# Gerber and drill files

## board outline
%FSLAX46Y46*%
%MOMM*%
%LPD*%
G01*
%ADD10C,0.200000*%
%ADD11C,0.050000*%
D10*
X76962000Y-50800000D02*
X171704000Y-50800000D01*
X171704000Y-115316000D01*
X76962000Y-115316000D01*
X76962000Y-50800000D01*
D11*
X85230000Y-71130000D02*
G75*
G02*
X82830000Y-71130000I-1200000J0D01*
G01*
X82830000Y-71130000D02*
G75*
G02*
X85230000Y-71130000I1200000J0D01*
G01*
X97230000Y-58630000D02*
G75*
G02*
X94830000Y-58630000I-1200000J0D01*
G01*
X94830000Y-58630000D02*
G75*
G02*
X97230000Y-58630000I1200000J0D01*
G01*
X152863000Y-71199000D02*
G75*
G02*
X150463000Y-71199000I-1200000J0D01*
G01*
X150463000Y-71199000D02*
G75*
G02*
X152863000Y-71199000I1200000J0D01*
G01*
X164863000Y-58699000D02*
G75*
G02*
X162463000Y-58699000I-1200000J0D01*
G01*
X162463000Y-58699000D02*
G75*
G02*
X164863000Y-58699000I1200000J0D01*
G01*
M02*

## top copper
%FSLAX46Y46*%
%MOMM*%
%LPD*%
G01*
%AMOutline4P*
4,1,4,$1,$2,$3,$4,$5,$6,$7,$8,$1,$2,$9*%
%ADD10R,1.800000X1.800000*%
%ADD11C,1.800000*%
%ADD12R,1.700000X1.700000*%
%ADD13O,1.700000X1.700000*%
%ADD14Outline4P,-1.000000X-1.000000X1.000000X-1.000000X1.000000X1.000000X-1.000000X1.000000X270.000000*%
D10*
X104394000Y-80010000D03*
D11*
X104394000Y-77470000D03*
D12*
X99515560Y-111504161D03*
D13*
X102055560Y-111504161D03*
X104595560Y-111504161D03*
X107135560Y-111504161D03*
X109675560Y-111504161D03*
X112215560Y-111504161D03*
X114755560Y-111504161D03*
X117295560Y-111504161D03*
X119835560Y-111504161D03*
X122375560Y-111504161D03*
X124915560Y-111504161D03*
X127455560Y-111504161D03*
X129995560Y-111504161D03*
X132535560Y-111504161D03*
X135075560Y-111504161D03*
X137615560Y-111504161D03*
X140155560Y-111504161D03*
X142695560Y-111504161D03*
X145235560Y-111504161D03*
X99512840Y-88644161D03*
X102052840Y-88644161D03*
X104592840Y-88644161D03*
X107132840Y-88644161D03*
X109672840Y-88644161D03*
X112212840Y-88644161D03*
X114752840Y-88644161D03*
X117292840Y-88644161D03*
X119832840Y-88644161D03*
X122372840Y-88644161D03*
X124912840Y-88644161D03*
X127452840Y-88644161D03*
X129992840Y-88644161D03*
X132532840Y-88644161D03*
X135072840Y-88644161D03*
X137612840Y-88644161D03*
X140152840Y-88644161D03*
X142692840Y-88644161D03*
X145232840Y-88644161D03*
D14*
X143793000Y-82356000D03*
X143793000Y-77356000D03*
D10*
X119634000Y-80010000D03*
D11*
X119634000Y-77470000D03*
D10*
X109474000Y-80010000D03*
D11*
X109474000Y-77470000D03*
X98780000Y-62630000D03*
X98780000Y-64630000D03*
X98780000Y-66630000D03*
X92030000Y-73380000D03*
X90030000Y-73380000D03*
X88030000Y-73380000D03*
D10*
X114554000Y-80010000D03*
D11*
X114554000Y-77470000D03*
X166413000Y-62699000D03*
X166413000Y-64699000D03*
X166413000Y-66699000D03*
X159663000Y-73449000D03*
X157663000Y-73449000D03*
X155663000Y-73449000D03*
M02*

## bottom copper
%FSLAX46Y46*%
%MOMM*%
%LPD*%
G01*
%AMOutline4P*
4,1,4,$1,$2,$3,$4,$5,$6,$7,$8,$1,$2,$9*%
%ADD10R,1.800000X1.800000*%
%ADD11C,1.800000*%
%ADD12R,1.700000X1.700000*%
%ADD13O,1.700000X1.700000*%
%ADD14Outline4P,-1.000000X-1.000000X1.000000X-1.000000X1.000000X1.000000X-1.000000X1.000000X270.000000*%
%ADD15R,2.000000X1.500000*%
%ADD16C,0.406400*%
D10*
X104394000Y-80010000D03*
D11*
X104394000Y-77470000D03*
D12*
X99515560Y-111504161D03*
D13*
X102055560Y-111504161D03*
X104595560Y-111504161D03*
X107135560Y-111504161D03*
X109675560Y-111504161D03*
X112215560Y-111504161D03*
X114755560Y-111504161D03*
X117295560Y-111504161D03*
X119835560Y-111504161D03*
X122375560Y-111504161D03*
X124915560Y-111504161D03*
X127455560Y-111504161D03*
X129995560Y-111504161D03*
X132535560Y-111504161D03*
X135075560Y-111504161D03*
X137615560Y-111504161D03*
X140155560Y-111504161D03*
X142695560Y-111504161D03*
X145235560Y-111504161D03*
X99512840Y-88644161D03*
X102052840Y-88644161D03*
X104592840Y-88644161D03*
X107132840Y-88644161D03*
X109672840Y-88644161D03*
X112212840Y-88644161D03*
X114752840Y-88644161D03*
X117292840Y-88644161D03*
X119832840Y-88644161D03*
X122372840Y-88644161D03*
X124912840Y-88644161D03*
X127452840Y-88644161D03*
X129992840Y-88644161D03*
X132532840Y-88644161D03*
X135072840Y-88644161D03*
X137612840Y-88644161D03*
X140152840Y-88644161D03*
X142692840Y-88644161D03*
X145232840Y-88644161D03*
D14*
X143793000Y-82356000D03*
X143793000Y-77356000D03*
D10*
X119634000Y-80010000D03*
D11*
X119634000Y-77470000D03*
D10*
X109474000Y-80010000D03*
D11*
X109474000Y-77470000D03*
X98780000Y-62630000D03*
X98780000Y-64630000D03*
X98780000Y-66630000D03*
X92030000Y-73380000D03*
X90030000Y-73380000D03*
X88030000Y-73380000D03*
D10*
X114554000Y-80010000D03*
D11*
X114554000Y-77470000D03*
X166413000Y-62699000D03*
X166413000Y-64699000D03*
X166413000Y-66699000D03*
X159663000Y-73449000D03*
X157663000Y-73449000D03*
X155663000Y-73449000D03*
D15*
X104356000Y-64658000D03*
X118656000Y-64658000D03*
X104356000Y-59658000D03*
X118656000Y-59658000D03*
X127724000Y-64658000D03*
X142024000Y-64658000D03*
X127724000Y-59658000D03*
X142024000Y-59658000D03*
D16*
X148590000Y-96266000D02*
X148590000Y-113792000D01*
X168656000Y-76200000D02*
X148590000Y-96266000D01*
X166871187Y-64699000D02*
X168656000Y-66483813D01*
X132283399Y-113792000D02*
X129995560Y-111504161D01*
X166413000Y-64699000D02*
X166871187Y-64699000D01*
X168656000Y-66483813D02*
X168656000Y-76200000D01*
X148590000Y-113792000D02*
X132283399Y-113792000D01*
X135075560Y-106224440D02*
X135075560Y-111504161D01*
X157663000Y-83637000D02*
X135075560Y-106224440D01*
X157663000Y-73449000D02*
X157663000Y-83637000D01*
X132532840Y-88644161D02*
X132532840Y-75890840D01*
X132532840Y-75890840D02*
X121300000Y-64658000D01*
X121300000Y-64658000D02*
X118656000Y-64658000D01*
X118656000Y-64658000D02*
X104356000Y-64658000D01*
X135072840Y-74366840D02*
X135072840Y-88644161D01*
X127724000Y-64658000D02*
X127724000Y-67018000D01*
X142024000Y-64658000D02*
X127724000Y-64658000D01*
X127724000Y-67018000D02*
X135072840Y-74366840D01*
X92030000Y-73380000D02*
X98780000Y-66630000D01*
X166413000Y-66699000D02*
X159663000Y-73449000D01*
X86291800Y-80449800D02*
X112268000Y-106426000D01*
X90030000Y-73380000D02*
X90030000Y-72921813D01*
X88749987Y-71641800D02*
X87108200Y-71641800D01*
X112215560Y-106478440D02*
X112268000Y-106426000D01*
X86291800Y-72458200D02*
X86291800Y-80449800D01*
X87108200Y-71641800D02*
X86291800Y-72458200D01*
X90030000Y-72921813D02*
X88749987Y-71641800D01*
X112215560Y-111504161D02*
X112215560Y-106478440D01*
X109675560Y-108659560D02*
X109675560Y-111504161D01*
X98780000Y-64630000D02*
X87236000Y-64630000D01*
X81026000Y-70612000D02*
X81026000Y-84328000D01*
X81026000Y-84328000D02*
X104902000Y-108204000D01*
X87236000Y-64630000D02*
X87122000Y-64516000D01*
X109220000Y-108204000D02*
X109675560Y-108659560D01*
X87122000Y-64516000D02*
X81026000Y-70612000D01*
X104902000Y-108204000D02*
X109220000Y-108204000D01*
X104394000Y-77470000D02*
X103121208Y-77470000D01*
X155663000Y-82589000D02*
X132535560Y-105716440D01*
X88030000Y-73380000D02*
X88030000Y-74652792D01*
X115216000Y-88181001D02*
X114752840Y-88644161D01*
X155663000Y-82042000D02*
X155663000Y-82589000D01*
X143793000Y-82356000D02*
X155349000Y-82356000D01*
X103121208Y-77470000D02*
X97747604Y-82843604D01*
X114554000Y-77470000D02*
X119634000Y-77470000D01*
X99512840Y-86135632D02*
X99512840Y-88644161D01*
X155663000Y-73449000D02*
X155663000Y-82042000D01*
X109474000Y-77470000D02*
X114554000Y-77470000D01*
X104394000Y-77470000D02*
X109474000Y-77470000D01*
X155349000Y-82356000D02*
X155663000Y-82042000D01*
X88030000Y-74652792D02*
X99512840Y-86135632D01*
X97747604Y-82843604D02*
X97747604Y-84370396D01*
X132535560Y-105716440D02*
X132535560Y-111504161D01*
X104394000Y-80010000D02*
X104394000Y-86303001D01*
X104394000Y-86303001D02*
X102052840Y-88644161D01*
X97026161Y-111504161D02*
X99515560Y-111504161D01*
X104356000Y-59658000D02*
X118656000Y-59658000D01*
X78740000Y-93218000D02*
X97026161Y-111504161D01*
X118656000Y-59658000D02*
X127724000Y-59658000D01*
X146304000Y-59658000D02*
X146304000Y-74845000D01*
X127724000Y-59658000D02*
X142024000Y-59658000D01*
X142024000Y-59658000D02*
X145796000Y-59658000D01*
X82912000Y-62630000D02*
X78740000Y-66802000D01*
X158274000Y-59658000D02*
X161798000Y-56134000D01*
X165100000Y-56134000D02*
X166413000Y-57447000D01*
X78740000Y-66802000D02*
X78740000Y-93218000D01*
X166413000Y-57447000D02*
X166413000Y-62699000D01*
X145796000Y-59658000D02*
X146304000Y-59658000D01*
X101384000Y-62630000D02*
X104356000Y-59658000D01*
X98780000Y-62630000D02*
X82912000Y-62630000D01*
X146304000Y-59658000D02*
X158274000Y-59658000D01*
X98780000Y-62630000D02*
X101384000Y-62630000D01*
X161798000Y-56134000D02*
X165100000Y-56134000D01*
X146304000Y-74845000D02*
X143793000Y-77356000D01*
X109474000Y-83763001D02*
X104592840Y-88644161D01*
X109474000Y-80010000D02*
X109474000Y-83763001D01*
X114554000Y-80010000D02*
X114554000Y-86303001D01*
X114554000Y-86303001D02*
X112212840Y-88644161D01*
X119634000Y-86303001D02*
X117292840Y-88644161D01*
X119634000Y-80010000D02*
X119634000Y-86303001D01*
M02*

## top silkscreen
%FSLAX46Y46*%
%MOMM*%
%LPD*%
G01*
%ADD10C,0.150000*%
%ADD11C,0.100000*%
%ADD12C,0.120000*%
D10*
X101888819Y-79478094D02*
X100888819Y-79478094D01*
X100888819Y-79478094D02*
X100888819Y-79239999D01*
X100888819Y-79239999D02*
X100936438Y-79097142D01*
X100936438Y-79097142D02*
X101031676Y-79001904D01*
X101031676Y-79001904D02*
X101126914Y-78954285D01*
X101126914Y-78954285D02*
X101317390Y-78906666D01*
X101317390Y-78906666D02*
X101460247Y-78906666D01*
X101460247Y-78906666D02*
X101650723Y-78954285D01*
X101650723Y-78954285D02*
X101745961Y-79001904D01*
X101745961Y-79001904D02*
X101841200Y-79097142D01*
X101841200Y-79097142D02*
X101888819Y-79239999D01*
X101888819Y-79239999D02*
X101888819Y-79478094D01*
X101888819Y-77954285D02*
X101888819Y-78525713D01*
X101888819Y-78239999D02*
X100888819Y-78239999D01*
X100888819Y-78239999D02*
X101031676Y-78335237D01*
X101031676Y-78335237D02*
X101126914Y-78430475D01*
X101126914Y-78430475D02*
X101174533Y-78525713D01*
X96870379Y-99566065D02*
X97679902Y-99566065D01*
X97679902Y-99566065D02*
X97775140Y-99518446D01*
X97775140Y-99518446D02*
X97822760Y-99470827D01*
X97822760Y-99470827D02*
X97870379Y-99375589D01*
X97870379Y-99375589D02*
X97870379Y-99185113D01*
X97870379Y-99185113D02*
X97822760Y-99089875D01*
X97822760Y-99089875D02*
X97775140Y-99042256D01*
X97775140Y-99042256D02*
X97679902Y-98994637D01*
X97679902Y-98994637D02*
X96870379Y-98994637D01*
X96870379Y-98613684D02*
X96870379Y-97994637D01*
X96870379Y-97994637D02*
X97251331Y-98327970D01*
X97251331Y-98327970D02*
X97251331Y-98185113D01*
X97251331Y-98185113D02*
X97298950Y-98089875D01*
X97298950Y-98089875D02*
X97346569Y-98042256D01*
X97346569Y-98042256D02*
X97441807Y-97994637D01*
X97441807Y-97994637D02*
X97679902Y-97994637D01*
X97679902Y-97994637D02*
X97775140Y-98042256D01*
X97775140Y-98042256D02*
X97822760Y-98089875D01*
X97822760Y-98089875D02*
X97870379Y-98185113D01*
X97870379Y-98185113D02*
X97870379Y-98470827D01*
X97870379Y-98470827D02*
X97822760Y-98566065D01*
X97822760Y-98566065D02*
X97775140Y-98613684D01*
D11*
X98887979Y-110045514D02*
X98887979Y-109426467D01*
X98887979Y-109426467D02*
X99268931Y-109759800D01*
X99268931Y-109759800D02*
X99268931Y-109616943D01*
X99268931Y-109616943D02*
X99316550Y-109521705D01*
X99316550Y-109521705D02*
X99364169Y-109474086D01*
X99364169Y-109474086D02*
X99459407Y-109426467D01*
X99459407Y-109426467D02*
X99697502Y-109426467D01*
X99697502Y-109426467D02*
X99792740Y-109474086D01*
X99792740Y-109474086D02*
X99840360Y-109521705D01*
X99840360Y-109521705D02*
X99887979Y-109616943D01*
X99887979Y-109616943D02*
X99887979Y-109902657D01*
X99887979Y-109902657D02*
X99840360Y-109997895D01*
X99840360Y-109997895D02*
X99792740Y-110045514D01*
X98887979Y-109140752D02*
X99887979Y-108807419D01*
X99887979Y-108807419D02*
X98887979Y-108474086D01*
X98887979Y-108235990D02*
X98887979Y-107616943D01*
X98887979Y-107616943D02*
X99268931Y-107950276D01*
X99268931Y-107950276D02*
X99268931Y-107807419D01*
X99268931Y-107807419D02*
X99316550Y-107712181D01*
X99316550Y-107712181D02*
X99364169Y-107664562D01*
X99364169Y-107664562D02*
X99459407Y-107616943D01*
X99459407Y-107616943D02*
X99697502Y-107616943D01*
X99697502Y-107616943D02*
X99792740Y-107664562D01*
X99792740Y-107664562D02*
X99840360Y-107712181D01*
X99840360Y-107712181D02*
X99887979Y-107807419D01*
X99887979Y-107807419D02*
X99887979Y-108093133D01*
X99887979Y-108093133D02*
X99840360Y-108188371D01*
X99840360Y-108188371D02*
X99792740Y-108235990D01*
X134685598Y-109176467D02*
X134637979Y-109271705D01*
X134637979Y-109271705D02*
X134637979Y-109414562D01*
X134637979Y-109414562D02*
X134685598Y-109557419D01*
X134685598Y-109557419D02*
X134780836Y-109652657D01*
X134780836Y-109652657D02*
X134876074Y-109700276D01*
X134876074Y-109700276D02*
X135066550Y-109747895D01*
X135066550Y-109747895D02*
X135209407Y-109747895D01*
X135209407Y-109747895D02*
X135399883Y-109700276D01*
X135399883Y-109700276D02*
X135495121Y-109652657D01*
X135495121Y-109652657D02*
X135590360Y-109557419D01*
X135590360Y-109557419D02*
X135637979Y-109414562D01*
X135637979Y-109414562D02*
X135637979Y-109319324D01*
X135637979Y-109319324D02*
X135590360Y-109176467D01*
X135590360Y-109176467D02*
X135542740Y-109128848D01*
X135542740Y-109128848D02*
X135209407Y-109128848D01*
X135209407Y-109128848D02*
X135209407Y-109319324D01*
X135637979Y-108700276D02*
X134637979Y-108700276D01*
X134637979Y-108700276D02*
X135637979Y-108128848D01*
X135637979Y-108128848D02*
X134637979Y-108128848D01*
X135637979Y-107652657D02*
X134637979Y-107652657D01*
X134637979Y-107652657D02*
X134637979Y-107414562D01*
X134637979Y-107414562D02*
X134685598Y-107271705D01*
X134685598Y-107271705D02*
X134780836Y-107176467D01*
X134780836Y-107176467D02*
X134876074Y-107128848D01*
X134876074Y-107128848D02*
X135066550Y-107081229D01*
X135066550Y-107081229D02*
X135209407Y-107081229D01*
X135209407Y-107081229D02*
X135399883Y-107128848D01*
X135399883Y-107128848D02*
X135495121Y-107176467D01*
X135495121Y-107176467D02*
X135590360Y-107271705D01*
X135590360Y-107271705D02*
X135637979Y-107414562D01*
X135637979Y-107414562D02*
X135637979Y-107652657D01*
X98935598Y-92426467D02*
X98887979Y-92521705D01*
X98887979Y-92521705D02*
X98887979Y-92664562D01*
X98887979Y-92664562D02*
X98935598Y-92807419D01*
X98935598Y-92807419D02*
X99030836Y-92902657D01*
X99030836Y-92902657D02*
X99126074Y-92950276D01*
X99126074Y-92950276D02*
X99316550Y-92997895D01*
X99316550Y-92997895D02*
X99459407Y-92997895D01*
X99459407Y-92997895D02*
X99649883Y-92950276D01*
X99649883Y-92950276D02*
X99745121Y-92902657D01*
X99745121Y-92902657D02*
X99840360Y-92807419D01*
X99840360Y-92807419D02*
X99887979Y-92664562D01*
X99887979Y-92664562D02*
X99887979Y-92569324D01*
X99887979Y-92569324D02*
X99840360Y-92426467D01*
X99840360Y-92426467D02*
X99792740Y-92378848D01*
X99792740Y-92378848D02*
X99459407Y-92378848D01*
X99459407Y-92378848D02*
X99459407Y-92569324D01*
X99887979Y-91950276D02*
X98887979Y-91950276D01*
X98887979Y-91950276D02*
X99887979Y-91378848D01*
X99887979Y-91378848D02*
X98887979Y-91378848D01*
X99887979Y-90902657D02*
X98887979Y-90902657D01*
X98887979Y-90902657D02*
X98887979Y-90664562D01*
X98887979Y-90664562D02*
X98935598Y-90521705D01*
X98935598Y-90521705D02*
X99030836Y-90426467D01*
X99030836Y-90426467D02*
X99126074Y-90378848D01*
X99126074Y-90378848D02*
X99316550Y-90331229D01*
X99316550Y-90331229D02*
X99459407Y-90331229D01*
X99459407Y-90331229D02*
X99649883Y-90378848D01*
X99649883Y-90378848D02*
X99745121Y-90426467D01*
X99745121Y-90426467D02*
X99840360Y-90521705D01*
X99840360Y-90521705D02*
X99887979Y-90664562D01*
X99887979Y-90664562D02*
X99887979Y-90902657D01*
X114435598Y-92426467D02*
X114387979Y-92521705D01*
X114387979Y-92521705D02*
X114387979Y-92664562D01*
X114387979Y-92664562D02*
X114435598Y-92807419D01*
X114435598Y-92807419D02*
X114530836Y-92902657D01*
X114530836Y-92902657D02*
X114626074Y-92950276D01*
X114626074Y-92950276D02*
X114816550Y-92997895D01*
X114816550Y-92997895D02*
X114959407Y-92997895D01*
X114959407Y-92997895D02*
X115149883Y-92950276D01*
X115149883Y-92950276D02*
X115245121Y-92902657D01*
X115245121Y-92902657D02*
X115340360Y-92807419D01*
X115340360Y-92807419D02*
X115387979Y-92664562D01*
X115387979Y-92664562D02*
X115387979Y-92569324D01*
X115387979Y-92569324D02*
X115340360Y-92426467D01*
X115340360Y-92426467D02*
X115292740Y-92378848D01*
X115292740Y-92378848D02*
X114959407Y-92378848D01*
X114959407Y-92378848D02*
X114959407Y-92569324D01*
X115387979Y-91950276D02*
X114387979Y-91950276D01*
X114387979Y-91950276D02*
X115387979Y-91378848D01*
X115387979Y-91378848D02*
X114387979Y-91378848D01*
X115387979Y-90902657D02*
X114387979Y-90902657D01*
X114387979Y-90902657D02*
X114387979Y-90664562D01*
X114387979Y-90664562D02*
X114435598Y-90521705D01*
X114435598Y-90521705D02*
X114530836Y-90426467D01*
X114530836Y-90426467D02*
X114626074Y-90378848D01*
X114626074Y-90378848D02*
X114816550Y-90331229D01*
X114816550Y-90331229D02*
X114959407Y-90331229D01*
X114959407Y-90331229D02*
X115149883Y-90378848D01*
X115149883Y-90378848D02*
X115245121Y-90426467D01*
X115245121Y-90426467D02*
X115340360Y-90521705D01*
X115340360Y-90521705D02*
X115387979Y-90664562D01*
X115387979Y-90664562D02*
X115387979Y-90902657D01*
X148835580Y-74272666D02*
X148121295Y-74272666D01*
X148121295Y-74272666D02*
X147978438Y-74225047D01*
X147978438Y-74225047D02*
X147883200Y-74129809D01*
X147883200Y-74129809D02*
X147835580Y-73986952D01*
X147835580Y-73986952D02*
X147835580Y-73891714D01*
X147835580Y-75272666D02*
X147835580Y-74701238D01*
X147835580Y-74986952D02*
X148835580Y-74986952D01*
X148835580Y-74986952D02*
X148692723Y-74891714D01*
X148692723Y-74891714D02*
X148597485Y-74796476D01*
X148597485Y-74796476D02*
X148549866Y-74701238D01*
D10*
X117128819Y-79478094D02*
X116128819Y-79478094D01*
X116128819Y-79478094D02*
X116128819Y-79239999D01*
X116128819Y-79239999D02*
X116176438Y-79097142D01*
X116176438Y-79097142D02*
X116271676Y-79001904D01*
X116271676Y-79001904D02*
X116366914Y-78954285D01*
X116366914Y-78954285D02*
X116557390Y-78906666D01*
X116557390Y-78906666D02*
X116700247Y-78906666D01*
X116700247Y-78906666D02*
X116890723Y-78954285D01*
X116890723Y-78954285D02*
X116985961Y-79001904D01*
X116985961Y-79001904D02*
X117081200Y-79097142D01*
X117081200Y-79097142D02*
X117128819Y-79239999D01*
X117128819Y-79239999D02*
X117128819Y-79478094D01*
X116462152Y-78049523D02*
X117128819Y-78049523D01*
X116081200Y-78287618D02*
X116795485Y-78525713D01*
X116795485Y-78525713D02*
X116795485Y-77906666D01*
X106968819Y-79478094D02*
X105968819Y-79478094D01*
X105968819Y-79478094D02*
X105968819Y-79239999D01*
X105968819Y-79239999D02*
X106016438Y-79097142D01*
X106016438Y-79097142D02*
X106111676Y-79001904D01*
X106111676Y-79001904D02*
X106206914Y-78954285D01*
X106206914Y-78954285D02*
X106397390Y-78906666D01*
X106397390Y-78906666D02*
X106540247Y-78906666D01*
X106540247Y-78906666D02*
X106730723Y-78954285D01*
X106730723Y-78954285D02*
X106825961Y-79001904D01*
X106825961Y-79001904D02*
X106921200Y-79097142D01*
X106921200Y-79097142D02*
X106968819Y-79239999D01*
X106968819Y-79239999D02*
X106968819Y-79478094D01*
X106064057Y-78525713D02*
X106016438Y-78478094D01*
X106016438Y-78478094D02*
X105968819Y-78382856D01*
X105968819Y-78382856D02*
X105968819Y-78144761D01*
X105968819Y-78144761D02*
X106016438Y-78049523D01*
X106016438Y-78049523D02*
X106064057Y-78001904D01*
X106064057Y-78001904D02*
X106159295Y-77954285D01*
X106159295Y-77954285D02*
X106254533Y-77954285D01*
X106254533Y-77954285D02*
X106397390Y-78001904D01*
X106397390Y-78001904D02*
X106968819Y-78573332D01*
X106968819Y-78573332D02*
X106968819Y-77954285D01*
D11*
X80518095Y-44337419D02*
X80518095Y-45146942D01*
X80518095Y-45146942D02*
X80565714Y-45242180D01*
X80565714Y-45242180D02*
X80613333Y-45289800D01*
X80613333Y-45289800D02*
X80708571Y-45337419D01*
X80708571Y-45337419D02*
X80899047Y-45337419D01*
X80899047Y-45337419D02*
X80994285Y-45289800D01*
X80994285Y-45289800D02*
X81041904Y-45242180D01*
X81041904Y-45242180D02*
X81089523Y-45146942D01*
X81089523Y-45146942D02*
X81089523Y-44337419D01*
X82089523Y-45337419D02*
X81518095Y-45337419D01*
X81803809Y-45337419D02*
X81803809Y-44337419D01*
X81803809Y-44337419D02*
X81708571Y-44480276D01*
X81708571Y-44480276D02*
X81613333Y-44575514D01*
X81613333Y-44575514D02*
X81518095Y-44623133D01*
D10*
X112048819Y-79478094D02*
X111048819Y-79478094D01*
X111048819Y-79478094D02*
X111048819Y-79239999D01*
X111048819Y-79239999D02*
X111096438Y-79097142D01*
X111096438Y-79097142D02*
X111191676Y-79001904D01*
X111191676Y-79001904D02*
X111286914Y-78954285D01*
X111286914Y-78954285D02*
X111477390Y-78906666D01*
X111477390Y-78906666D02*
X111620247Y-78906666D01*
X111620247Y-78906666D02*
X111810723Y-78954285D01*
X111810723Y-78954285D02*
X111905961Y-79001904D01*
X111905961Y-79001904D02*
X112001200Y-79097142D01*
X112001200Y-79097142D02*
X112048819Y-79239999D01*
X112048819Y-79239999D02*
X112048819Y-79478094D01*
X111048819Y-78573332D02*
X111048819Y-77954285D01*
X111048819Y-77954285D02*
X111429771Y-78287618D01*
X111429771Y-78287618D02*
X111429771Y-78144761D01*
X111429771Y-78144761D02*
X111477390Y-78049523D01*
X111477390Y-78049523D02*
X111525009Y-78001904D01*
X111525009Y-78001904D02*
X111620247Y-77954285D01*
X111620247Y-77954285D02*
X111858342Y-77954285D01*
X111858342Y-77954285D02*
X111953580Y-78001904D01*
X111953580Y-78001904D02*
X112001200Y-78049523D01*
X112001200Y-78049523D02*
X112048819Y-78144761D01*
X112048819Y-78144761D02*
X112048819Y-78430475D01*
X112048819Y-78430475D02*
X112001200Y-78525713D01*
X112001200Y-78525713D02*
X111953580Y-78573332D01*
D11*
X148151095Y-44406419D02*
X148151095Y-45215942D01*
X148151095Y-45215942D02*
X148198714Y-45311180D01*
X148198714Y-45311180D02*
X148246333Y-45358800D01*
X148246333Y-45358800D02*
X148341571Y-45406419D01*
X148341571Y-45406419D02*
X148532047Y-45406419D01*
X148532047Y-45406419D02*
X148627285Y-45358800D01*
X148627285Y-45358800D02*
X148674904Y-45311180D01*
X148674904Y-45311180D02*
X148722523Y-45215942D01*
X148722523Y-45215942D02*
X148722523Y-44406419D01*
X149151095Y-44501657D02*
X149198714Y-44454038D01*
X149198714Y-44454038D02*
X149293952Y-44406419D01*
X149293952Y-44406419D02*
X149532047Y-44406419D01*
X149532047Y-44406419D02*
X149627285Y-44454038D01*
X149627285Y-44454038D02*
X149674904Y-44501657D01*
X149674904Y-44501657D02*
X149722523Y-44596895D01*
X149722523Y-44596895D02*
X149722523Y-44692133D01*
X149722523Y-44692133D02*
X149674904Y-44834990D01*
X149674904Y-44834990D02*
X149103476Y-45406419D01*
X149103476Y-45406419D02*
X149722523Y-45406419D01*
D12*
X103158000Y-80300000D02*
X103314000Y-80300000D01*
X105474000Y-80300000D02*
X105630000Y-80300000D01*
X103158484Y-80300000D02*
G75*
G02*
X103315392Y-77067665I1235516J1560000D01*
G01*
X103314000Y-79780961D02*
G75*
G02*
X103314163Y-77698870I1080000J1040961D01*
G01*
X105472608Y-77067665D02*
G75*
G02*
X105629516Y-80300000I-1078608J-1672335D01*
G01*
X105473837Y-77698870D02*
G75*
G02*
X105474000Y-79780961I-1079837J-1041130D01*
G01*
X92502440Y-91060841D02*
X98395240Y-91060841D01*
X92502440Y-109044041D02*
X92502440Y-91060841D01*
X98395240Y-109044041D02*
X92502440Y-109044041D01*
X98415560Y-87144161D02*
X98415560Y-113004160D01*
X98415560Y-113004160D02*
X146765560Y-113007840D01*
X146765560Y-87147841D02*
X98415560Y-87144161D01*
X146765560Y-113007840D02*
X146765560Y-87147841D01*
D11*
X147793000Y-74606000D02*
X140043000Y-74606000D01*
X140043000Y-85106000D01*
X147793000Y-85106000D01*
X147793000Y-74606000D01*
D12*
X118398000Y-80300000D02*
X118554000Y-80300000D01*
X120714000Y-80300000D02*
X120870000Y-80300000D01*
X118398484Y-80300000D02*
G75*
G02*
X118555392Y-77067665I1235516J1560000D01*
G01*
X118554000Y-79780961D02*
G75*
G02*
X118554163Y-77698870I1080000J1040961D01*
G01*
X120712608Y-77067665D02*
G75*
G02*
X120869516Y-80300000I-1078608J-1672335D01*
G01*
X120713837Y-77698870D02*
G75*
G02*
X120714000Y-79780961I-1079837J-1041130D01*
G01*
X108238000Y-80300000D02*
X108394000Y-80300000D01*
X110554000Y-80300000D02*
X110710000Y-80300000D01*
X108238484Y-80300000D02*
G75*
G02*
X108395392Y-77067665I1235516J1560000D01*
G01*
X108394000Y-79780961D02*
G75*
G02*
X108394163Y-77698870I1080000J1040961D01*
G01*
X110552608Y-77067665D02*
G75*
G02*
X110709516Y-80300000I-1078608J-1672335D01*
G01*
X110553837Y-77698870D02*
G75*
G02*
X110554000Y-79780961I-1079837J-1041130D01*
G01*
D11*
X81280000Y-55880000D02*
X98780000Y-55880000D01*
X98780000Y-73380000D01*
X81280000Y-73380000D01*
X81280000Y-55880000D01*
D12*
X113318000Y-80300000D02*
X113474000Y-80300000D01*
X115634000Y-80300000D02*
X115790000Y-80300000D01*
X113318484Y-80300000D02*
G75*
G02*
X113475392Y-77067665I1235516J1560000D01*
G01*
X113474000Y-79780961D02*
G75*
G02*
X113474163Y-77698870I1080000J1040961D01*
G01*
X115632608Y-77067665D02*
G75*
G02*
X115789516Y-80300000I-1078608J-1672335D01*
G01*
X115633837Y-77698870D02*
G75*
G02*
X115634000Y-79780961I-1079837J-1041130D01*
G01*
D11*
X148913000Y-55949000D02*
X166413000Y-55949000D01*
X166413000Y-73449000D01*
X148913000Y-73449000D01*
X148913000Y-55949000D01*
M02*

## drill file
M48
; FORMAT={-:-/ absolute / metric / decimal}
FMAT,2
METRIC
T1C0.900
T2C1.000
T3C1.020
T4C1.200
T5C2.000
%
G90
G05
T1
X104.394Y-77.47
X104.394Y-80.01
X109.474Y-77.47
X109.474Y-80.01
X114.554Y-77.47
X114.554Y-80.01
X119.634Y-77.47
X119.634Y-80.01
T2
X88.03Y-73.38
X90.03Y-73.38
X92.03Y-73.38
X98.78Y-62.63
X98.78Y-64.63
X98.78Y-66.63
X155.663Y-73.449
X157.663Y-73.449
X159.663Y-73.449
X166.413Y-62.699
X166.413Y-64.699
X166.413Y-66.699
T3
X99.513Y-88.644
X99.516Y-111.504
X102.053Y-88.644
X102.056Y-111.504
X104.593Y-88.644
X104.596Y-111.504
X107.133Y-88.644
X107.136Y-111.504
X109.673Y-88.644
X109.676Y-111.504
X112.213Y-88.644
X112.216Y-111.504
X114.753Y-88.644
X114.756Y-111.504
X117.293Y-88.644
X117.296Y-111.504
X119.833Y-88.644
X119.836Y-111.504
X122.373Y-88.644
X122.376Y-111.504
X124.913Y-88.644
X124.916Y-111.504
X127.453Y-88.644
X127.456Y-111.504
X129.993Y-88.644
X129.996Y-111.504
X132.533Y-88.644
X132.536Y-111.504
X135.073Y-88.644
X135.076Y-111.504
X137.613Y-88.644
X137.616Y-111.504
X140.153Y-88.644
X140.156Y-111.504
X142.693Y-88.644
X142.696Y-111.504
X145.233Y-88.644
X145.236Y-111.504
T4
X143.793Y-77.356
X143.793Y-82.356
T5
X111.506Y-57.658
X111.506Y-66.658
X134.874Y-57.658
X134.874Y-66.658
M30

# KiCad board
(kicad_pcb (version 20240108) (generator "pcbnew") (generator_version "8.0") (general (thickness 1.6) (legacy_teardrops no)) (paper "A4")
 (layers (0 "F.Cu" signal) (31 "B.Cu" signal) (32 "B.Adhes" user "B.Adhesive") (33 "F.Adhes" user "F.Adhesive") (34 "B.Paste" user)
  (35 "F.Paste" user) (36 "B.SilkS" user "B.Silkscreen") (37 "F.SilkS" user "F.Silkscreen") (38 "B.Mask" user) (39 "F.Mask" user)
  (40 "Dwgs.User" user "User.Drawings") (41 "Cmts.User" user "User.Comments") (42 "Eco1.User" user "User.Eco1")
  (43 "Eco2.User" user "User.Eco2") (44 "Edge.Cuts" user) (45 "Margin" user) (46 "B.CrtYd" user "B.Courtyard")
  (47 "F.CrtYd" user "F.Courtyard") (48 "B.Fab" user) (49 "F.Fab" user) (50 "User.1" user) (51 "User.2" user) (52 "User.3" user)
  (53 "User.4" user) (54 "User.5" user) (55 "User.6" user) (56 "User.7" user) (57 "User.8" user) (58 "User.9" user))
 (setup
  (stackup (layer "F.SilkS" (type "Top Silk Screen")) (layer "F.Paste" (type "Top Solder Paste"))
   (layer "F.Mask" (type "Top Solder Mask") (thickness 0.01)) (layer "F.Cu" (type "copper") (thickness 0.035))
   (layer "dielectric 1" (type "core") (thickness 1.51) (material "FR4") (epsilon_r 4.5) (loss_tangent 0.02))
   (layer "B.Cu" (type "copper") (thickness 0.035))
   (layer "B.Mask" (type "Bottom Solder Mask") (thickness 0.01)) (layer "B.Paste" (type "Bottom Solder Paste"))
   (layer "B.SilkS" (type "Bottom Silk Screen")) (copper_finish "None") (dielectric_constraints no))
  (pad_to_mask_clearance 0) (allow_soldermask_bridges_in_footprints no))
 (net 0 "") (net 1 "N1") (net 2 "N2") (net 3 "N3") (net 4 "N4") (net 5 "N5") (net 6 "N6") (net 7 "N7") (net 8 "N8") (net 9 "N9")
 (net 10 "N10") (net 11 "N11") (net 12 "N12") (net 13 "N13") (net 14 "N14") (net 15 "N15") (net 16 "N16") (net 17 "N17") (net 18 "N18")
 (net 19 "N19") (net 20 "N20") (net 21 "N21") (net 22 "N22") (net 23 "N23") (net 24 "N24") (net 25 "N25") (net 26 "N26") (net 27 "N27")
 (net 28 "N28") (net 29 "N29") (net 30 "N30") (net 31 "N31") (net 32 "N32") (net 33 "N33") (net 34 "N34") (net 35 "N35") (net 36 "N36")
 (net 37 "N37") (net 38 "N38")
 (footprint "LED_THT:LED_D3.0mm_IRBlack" (layer "F.Cu") (at 104.394 80.01 90)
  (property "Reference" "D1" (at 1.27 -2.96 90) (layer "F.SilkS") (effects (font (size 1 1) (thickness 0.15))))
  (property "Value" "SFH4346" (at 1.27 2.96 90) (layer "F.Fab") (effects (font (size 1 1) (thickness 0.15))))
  (fp_line (start -0.29 -1.236) (end -0.29 -1.08) (stroke (width 0.12) (type solid)) (layer "F.SilkS"))
  (fp_line (start -0.29 1.08) (end -0.29 1.236) (stroke (width 0.12) (type solid)) (layer "F.SilkS"))
  (fp_arc (start -0.29 -1.235516) (mid 1.366487 -1.987659) (end 2.942335 -1.078608) (stroke (width 0.12) (type solid)) (layer "F.SilkS"))
  (fp_arc (start 0.229039 -1.08) (mid 1.270117 -1.5) (end 2.31113 -1.079837) (stroke (width 0.12) (type solid)) (layer "F.SilkS"))
  (fp_arc (start 2.942335 1.078608) (mid 1.366487 1.987659) (end -0.29 1.235516) (stroke (width 0.12) (type solid)) (layer "F.SilkS"))
  (fp_arc (start 2.31113 1.079837) (mid 1.270117 1.5) (end 0.229039 1.08) (stroke (width 0.12) (type solid)) (layer "F.SilkS"))
  (pad "1" thru_hole rect (at 0 0 90) (size 1.8 1.8) (drill 0.9) (layers "*.Cu" "*.Mask") (remove_unused_layers no) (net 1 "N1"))
  (pad "2" thru_hole circle (at 2.54 0 90) (size 1.8 1.8) (drill 0.9) (layers "*.Cu" "*.Mask") (remove_unused_layers no) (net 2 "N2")))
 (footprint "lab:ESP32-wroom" (layer "F.Cu") (at 99.51556 111.504161 90)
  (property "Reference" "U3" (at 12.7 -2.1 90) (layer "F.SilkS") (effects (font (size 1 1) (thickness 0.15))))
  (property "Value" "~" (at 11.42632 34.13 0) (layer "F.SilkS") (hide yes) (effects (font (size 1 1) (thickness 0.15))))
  (fp_line (start 20.44332 -7.01312) (end 20.44332 -1.12032) (stroke (width 0.12) (type solid)) (layer "F.SilkS"))
  (fp_line (start 2.46012 -7.01312) (end 20.44332 -7.01312) (stroke (width 0.12) (type solid)) (layer "F.SilkS"))
  (fp_line (start 2.46012 -1.12032) (end 2.46012 -7.01312) (stroke (width 0.12) (type solid)) (layer "F.SilkS"))
  (fp_line (start 24.36 -1.1) (end -1.499999 -1.1) (stroke (width 0.12) (type solid)) (layer "F.SilkS"))
  (fp_line (start -1.499999 -1.1) (end -1.503679 47.25) (stroke (width 0.12) (type solid)) (layer "F.SilkS"))
  (fp_line (start 24.35632 47.25) (end 24.36 -1.1) (stroke (width 0.12) (type solid)) (layer "F.SilkS"))
  (fp_line (start -1.503679 47.25) (end 24.35632 47.25) (stroke (width 0.12) (type solid)) (layer "F.SilkS"))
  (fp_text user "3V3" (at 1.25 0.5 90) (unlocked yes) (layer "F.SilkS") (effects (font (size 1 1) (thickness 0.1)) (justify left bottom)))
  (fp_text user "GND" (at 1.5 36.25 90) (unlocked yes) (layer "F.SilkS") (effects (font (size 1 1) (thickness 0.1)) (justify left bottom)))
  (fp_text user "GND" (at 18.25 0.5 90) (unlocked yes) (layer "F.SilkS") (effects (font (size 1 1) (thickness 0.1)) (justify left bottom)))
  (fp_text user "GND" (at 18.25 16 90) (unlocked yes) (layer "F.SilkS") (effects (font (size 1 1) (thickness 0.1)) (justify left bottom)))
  (pad "1" thru_hole rect (at 0 0) (size 1.7 1.7) (drill 1.02) (layers "*.Cu" "*.Mask") (remove_unused_layers no) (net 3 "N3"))
  (pad "2" thru_hole oval (at 0 2.54) (size 1.7 1.7) (drill 1.02) (layers "*.Cu" "*.Mask") (remove_unused_layers no) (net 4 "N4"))
  (pad "3" thru_hole oval (at 0 5.08) (size 1.7 1.7) (drill 1.02) (layers "*.Cu" "*.Mask") (remove_unused_layers no) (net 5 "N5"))
  (pad "4" thru_hole oval (at 0 7.62) (size 1.7 1.7) (drill 1.02) (layers "*.Cu" "*.Mask") (remove_unused_layers no) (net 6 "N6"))
  (pad "5" thru_hole oval (at 0 10.16) (size 1.7 1.7) (drill 1.02) (layers "*.Cu" "*.Mask") (remove_unused_layers no) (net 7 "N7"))
  (pad "6" thru_hole oval (at 0 12.7) (size 1.7 1.7) (drill 1.02) (layers "*.Cu" "*.Mask") (remove_unused_layers no) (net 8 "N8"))
  (pad "7" thru_hole oval (at 0 15.24) (size 1.7 1.7) (drill 1.02) (layers "*.Cu" "*.Mask") (remove_unused_layers no) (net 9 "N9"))
  (pad "8" thru_hole oval (at 0 17.78) (size 1.7 1.7) (drill 1.02) (layers "*.Cu" "*.Mask") (remove_unused_layers no) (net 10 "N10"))
  (pad "9" thru_hole oval (at 0 20.32) (size 1.7 1.7) (drill 1.02) (layers "*.Cu" "*.Mask") (remove_unused_layers no) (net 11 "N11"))
  (pad "10" thru_hole oval (at 0 22.86) (size 1.7 1.7) (drill 1.02) (layers "*.Cu" "*.Mask") (remove_unused_layers no) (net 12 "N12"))
  (pad "11" thru_hole oval (at 0 25.4) (size 1.7 1.7) (drill 1.02) (layers "*.Cu" "*.Mask") (remove_unused_layers no) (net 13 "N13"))
  (pad "12" thru_hole oval (at 0 27.94) (size 1.7 1.7) (drill 1.02) (layers "*.Cu" "*.Mask") (remove_unused_layers no) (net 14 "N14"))
  (pad "13" thru_hole oval (at 0 30.48) (size 1.7 1.7) (drill 1.02) (layers "*.Cu" "*.Mask") (remove_unused_layers no) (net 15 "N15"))
  (pad "14" thru_hole oval (at 0 33.02) (size 1.7 1.7) (drill 1.02) (layers "*.Cu" "*.Mask") (remove_unused_layers no) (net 2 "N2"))
  (pad "15" thru_hole oval (at 0 35.56) (size 1.7 1.7) (drill 1.02) (layers "*.Cu" "*.Mask") (remove_unused_layers no) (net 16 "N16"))
  (pad "16" thru_hole oval (at 0 38.1) (size 1.7 1.7) (drill 1.02) (layers "*.Cu" "*.Mask") (remove_unused_layers no) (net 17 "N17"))
  (pad "17" thru_hole oval (at 0 40.64) (size 1.7 1.7) (drill 1.02) (layers "*.Cu" "*.Mask") (remove_unused_layers no) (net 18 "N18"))
  (pad "18" thru_hole oval (at 0 43.18) (size 1.7 1.7) (drill 1.02) (layers "*.Cu" "*.Mask") (remove_unused_layers no) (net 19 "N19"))
  (pad "19" thru_hole oval (at 0 45.72) (size 1.7 1.7) (drill 1.02) (layers "*.Cu" "*.Mask") (remove_unused_layers no) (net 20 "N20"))
  (pad "20" thru_hole oval (at 22.86 -0.00272) (size 1.7 1.7) (drill 1.02) (layers "*.Cu" "*.Mask") (remove_unused_layers no) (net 2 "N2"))
  (pad "21" thru_hole oval (at 22.86 2.53728) (size 1.7 1.7) (drill 1.02) (layers "*.Cu" "*.Mask") (remove_unused_layers no) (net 1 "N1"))
  (pad "22" thru_hole oval (at 22.86 5.07728) (size 1.7 1.7) (drill 1.02) (layers "*.Cu" "*.Mask") (remove_unused_layers no) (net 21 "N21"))
  (pad "23" thru_hole oval (at 22.86 7.61728) (size 1.7 1.7) (drill 1.02) (layers "*.Cu" "*.Mask") (remove_unused_layers no) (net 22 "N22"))
  (pad "24" thru_hole oval (at 22.86 10.15728) (size 1.7 1.7) (drill 1.02) (layers "*.Cu" "*.Mask") (remove_unused_layers no) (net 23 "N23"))
  (pad "25" thru_hole oval (at 22.86 12.69728) (size 1.7 1.7) (drill 1.02) (layers "*.Cu" "*.Mask") (remove_unused_layers no) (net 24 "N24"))
  (pad "26" thru_hole oval (at 22.86 15.23728) (size 1.7 1.7) (drill 1.02) (layers "*.Cu" "*.Mask") (remove_unused_layers no) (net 2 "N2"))
  (pad "27" thru_hole oval (at 22.86 17.77728) (size 1.7 1.7) (drill 1.02) (layers "*.Cu" "*.Mask") (remove_unused_layers no) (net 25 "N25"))
  (pad "28" thru_hole oval (at 22.86 20.31728) (size 1.7 1.7) (drill 1.02) (layers "*.Cu" "*.Mask") (remove_unused_layers no) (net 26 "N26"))
  (pad "29" thru_hole oval (at 22.86 22.85728) (size 1.7 1.7) (drill 1.02) (layers "*.Cu" "*.Mask") (remove_unused_layers no) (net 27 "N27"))
  (pad "30" thru_hole oval (at 22.86 25.39728) (size 1.7 1.7) (drill 1.02) (layers "*.Cu" "*.Mask") (remove_unused_layers no) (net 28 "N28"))
  (pad "31" thru_hole oval (at 22.86 27.93728) (size 1.7 1.7) (drill 1.02) (layers "*.Cu" "*.Mask") (remove_unused_layers no) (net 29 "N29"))
  (pad "32" thru_hole oval (at 22.86 30.47728) (size 1.7 1.7) (drill 1.02) (layers "*.Cu" "*.Mask") (remove_unused_layers no) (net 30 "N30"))
  (pad "33" thru_hole oval (at 22.86 33.01728) (size 1.7 1.7) (drill 1.02) (layers "*.Cu" "*.Mask") (remove_unused_layers no) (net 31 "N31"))
  (pad "34" thru_hole oval (at 22.86 35.55728) (size 1.7 1.7) (drill 1.02) (layers "*.Cu" "*.Mask") (remove_unused_layers no) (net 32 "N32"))
  (pad "35" thru_hole oval (at 22.86 38.09728) (size 1.7 1.7) (drill 1.02) (layers "*.Cu" "*.Mask") (remove_unused_layers no) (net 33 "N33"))
  (pad "36" thru_hole oval (at 22.86 40.63728) (size 1.7 1.7) (drill 1.02) (layers "*.Cu" "*.Mask") (remove_unused_layers no) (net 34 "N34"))
  (pad "37" thru_hole oval (at 22.86 43.17728) (size 1.7 1.7) (drill 1.02) (layers "*.Cu" "*.Mask") (remove_unused_layers no) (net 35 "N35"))
  (pad "38" thru_hole oval (at 22.86 45.71728) (size 1.7 1.7) (drill 1.02) (layers "*.Cu" "*.Mask") (remove_unused_layers no) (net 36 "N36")))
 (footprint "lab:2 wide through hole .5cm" (layer "F.Cu") (at 147.793 74.606 -90)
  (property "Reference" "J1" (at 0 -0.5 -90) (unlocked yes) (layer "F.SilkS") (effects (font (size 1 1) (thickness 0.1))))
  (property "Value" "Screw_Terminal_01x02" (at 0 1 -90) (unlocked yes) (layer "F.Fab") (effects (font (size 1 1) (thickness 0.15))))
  (fp_rect (start 0 0) (end 10.5 7.75) (stroke (width 0.1) (type default)) (fill none) (layer "F.SilkS"))
  (pad "1" thru_hole trapezoid (at 7.75 4 270) (size 2 2) (drill 1.2) (layers "*.Cu" "*.Mask" "Eco1.User") (remove_unused_layers no)
   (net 2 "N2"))
  (pad "2" thru_hole trapezoid (at 2.75 4 270) (size 2 2) (drill 1.2) (layers "*.Cu" "*.Mask") (remove_unused_layers no) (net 3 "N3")))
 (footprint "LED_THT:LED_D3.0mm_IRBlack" (layer "F.Cu") (at 119.634 80.01 90)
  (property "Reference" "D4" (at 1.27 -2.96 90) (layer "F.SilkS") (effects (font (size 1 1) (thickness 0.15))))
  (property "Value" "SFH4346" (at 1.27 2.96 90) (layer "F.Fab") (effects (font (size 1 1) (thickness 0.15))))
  (fp_line (start -0.29 -1.236) (end -0.29 -1.08) (stroke (width 0.12) (type solid)) (layer "F.SilkS"))
  (fp_line (start -0.29 1.08) (end -0.29 1.236) (stroke (width 0.12) (type solid)) (layer "F.SilkS"))
  (fp_arc (start -0.29 -1.235516) (mid 1.366487 -1.987659) (end 2.942335 -1.078608) (stroke (width 0.12) (type solid)) (layer "F.SilkS"))
  (fp_arc (start 0.229039 -1.08) (mid 1.270117 -1.5) (end 2.31113 -1.079837) (stroke (width 0.12) (type solid)) (layer "F.SilkS"))
  (fp_arc (start 2.942335 1.078608) (mid 1.366487 1.987659) (end -0.29 1.235516) (stroke (width 0.12) (type solid)) (layer "F.SilkS"))
  (fp_arc (start 2.31113 1.079837) (mid 1.270117 1.5) (end 0.229039 1.08) (stroke (width 0.12) (type solid)) (layer "F.SilkS"))
  (pad "1" thru_hole rect (at 0 0 90) (size 1.8 1.8) (drill 0.9) (layers "*.Cu" "*.Mask") (remove_unused_layers no) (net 25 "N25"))
  (pad "2" thru_hole circle (at 2.54 0 90) (size 1.8 1.8) (drill 0.9) (layers "*.Cu" "*.Mask") (remove_unused_layers no) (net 2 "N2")))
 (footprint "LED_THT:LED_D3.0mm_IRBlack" (layer "F.Cu") (at 109.474 80.01 90)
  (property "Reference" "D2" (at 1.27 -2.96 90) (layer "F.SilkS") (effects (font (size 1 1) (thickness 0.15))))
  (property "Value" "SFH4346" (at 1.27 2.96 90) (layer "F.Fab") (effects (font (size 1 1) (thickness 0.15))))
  (fp_line (start -0.29 -1.236) (end -0.29 -1.08) (stroke (width 0.12) (type solid)) (layer "F.SilkS"))
  (fp_line (start -0.29 1.08) (end -0.29 1.236) (stroke (width 0.12) (type solid)) (layer "F.SilkS"))
  (fp_arc (start -0.29 -1.235516) (mid 1.366487 -1.987659) (end 2.942335 -1.078608) (stroke (width 0.12) (type solid)) (layer "F.SilkS"))
  (fp_arc (start 0.229039 -1.08) (mid 1.270117 -1.5) (end 2.31113 -1.079837) (stroke (width 0.12) (type solid)) (layer "F.SilkS"))
  (fp_arc (start 2.942335 1.078608) (mid 1.366487 1.987659) (end -0.29 1.235516) (stroke (width 0.12) (type solid)) (layer "F.SilkS"))
  (fp_arc (start 2.31113 1.079837) (mid 1.270117 1.5) (end 0.229039 1.08) (stroke (width 0.12) (type solid)) (layer "F.SilkS"))
  (pad "1" thru_hole rect (at 0 0 90) (size 1.8 1.8) (drill 0.9) (layers "*.Cu" "*.Mask") (remove_unused_layers no) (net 21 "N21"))
  (pad "2" thru_hole circle (at 2.54 0 90) (size 1.8 1.8) (drill 0.9) (layers "*.Cu" "*.Mask") (remove_unused_layers no) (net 2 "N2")))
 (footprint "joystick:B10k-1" (layer "F.Cu") (at 81.28 55.88)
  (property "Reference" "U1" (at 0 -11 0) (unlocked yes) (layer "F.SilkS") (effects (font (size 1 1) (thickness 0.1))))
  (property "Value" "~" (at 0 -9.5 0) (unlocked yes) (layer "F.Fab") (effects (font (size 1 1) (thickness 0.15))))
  (fp_rect (start 0 0) (end 17.5 17.5) (stroke (width 0.1) (type default)) (fill none) (layer "F.SilkS"))
  (fp_circle (center 2.75 15.25) (end 3.95 15.25) (stroke (width 0.05) (type default)) (fill none) (layer "Edge.Cuts"))
  (fp_circle (center 14.75 2.75) (end 15.95 2.75) (stroke (width 0.05) (type default)) (fill none) (layer "Edge.Cuts"))
  (pad "1" thru_hole circle (at 17.5 6.75) (size 1.8 1.8) (drill 1) (layers "*.Cu" "*.Mask") (remove_unused_layers no) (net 3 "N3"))
  (pad "2" thru_hole circle (at 17.5 8.75) (size 1.8 1.8) (drill 1) (layers "*.Cu" "*.Mask") (remove_unused_layers no) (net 7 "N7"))
  (pad "3" thru_hole circle (at 17.5 10.75) (size 1.8 1.8) (drill 1) (layers "*.Cu" "*.Mask") (remove_unused_layers no) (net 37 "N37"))
  (pad "4" thru_hole circle (at 10.75 17.5) (size 1.8 1.8) (drill 1) (layers "*.Cu" "*.Mask") (remove_unused_layers no) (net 37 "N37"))
  (pad "5" thru_hole circle (at 8.75 17.5) (size 1.8 1.8) (drill 1) (layers "*.Cu" "*.Mask") (remove_unused_layers no) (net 8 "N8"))
  (pad "6" thru_hole circle (at 6.75 17.5) (size 1.8 1.8) (drill 1) (layers "*.Cu" "*.Mask") (remove_unused_layers no) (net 2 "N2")))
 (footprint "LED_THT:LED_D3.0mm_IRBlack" (layer "F.Cu") (at 114.554 80.01 90)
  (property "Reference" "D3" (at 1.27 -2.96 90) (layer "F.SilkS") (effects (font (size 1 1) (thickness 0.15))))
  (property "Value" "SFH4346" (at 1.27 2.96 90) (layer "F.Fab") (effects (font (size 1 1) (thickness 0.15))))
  (fp_line (start -0.29 -1.236) (end -0.29 -1.08) (stroke (width 0.12) (type solid)) (layer "F.SilkS"))
  (fp_line (start -0.29 1.08) (end -0.29 1.236) (stroke (width 0.12) (type solid)) (layer "F.SilkS"))
  (fp_arc (start -0.29 -1.235516) (mid 1.366487 -1.987659) (end 2.942335 -1.078608) (stroke (width 0.12) (type solid)) (layer "F.SilkS"))
  (fp_arc (start 0.229039 -1.08) (mid 1.270117 -1.5) (end 2.31113 -1.079837) (stroke (width 0.12) (type solid)) (layer "F.SilkS"))
  (fp_arc (start 2.942335 1.078608) (mid 1.366487 1.987659) (end -0.29 1.235516) (stroke (width 0.12) (type solid)) (layer "F.SilkS"))
  (fp_arc (start 2.31113 1.079837) (mid 1.270117 1.5) (end 0.229039 1.08) (stroke (width 0.12) (type solid)) (layer "F.SilkS"))
  (pad "1" thru_hole rect (at 0 0 90) (size 1.8 1.8) (drill 0.9) (layers "*.Cu" "*.Mask") (remove_unused_layers no) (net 24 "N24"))
  (pad "2" thru_hole circle (at 2.54 0 90) (size 1.8 1.8) (drill 0.9) (layers "*.Cu" "*.Mask") (remove_unused_layers no) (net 2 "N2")))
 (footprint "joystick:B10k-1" (layer "F.Cu") (at 148.913 55.949)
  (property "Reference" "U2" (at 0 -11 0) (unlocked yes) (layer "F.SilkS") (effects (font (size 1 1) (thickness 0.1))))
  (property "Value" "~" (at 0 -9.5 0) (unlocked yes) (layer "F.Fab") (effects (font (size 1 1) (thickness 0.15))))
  (fp_rect (start 0 0) (end 17.5 17.5) (stroke (width 0.1) (type default)) (fill none) (layer "F.SilkS"))
  (fp_circle (center 2.75 15.25) (end 3.95 15.25) (stroke (width 0.05) (type default)) (fill none) (layer "Edge.Cuts"))
  (fp_circle (center 14.75 2.75) (end 15.95 2.75) (stroke (width 0.05) (type default)) (fill none) (layer "Edge.Cuts"))
  (pad "1" thru_hole circle (at 17.5 6.75) (size 1.8 1.8) (drill 1) (layers "*.Cu" "*.Mask") (remove_unused_layers no) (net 3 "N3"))
  (pad "2" thru_hole circle (at 17.5 8.75) (size 1.8 1.8) (drill 1) (layers "*.Cu" "*.Mask") (remove_unused_layers no) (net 15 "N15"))
  (pad "3" thru_hole circle (at 17.5 10.75) (size 1.8 1.8) (drill 1) (layers "*.Cu" "*.Mask") (remove_unused_layers no) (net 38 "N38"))
  (pad "4" thru_hole circle (at 10.75 17.5) (size 1.8 1.8) (drill 1) (layers "*.Cu" "*.Mask") (remove_unused_layers no) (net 38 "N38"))
  (pad "5" thru_hole circle (at 8.75 17.5) (size 1.8 1.8) (drill 1) (layers "*.Cu" "*.Mask") (remove_unused_layers no) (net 16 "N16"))
  (pad "6" thru_hole circle (at 6.75 17.5) (size 1.8 1.8) (drill 1) (layers "*.Cu" "*.Mask") (remove_unused_layers no) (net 2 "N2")))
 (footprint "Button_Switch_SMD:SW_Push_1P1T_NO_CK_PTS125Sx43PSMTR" (layer "B.Cu") (at 111.506 62.158)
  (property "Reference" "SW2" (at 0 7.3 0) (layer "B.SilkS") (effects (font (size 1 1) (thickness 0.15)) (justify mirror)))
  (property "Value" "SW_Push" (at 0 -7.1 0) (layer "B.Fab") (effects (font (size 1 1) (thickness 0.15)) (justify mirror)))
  (pad "" np_thru_hole circle (at 0 -4.5) (size 2 2) (drill 2) (layers "*.Cu" "*.Mask"))
  (pad "" np_thru_hole circle (at 0 4.5) (size 2 2) (drill 2) (layers "*.Cu" "*.Mask"))
  (pad "1" smd rect (at -7.15 2.5) (size 2 1.5) (layers "B.Cu" "B.Paste" "B.Mask") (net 31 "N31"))
  (pad "1" smd rect (at 7.15 2.5) (size 2 1.5) (layers "B.Cu" "B.Paste" "B.Mask") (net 31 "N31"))
  (pad "2" smd rect (at -7.15 -2.5) (size 2 1.5) (layers "B.Cu" "B.Paste" "B.Mask") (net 3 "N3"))
  (pad "2" smd rect (at 7.15 -2.5) (size 2 1.5) (layers "B.Cu" "B.Paste" "B.Mask") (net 3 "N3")))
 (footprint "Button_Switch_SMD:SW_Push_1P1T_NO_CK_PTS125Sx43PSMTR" (layer "B.Cu") (at 134.874 62.158)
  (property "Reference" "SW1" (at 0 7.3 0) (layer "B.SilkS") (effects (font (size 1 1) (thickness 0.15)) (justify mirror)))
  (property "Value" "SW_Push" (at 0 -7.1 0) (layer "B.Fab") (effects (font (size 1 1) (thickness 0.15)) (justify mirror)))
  (pad "" np_thru_hole circle (at 0 -4.5) (size 2 2) (drill 2) (layers "*.Cu" "*.Mask"))
  (pad "" np_thru_hole circle (at 0 4.5) (size 2 2) (drill 2) (layers "*.Cu" "*.Mask"))
  (pad "1" smd rect (at -7.15 2.5) (size 2 1.5) (layers "B.Cu" "B.Paste" "B.Mask") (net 32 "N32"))
  (pad "1" smd rect (at 7.15 2.5) (size 2 1.5) (layers "B.Cu" "B.Paste" "B.Mask") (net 32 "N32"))
  (pad "2" smd rect (at -7.15 -2.5) (size 2 1.5) (layers "B.Cu" "B.Paste" "B.Mask") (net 3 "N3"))
  (pad "2" smd rect (at 7.15 -2.5) (size 2 1.5) (layers "B.Cu" "B.Paste" "B.Mask") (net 3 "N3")))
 (gr_rect (start 76.962 50.8) (end 171.704 115.316) (stroke (width 0.2) (type default)) (fill none) (layer "Edge.Cuts"))
 (segment (start 132.53284 88.644161) (end 132.53284 75.89084) (width 0.4064) (layer "B.Cu") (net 31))
 (segment (start 132.53284 75.89084) (end 121.3 64.658) (width 0.4064) (layer "B.Cu") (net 31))
 (segment (start 121.3 64.658) (end 118.656 64.658) (width 0.4064) (layer "B.Cu") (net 31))
 (segment (start 118.656 64.658) (end 104.356 64.658) (width 0.4064) (layer "B.Cu") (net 31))
 (segment (start 135.07284 74.36684) (end 135.07284 88.644161) (width 0.4064) (layer "B.Cu") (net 32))
 (segment (start 127.724 64.658) (end 127.724 67.018) (width 0.4064) (layer "B.Cu") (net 32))
 (segment (start 142.024 64.658) (end 127.724 64.658) (width 0.4064) (layer "B.Cu") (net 32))
 (segment (start 127.724 67.018) (end 135.07284 74.36684) (width 0.4064) (layer "B.Cu") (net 32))
 (segment (start 92.03 73.38) (end 98.78 66.63) (width 0.4064) (layer "B.Cu") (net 37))
 (segment (start 166.413 66.699) (end 159.663 73.449) (width 0.4064) (layer "B.Cu") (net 38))
 (segment (start 86.2918 80.4498) (end 112.268 106.426) (width 0.4064) (layer "B.Cu") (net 8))
 (segment (start 90.03 73.38) (end 90.03 72.921813) (width 0.4064) (layer "B.Cu") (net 8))
 (segment (start 88.749987 71.6418) (end 87.1082 71.6418) (width 0.4064) (layer "B.Cu") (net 8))
 (segment (start 112.21556 106.47844) (end 112.268 106.426) (width 0.4064) (layer "B.Cu") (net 8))
 (segment (start 86.2918 72.4582) (end 86.2918 80.4498) (width 0.4064) (layer "B.Cu") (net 8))
 (segment (start 87.1082 71.6418) (end 86.2918 72.4582) (width 0.4064) (layer "B.Cu") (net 8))
 (segment (start 90.03 72.921813) (end 88.749987 71.6418) (width 0.4064) (layer "B.Cu") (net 8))
 (segment (start 112.21556 111.504161) (end 112.21556 106.47844) (width 0.4064) (layer "B.Cu") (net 8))
 (segment (start 109.67556 108.65956) (end 109.67556 111.504161) (width 0.4064) (layer "B.Cu") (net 7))
 (segment (start 98.78 64.63) (end 87.236 64.63) (width 0.4064) (layer "B.Cu") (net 7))
 (segment (start 81.026 70.612) (end 81.026 84.328) (width 0.4064) (layer "B.Cu") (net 7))
 (segment (start 81.026 84.328) (end 104.902 108.204) (width 0.4064) (layer "B.Cu") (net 7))
 (segment (start 87.236 64.63) (end 87.122 64.516) (width 0.4064) (layer "B.Cu") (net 7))
 (segment (start 109.22 108.204) (end 109.67556 108.65956) (width 0.4064) (layer "B.Cu") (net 7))
 (segment (start 87.122 64.516) (end 81.026 70.612) (width 0.4064) (layer "B.Cu") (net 7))
 (segment (start 104.902 108.204) (end 109.22 108.204) (width 0.4064) (layer "B.Cu") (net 7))
 (segment (start 104.394 77.47) (end 103.121208 77.47) (width 0.4064) (layer "B.Cu") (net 2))
 (segment (start 155.663 82.589) (end 132.53556 105.71644) (width 0.4064) (layer "B.Cu") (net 2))
 (segment (start 88.03 73.38) (end 88.03 74.652792) (width 0.4064) (layer "B.Cu") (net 2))
 (segment (start 115.216 88.181001) (end 114.75284 88.644161) (width 0.4064) (layer "B.Cu") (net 2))
 (segment (start 155.663 82.042) (end 155.663 82.589) (width 0.4064) (layer "B.Cu") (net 2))
 (segment (start 143.793 82.356) (end 155.349 82.356) (width 0.4064) (layer "B.Cu") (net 2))
 (segment (start 103.121208 77.47) (end 97.747604 82.843604) (width 0.4064) (layer "B.Cu") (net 2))
 (segment (start 114.554 77.47) (end 119.634 77.47) (width 0.4064) (layer "B.Cu") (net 2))
 (segment (start 99.51284 86.135632) (end 99.51284 88.644161) (width 0.4064) (layer "B.Cu") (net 2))
 (segment (start 155.663 73.449) (end 155.663 82.042) (width 0.4064) (layer "B.Cu") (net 2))
 (segment (start 109.474 77.47) (end 114.554 77.47) (width 0.4064) (layer "B.Cu") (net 2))
 (segment (start 104.394 77.47) (end 109.474 77.47) (width 0.4064) (layer "B.Cu") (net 2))
 (segment (start 155.349 82.356) (end 155.663 82.042) (width 0.4064) (layer "B.Cu") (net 2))
 (segment (start 88.03 74.652792) (end 99.51284 86.135632) (width 0.4064) (layer "B.Cu") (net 2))
 (segment (start 97.747604 82.843604) (end 97.747604 84.370396) (width 0.4064) (layer "B.Cu") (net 2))
 (segment (start 132.53556 105.71644) (end 132.53556 111.504161) (width 0.4064) (layer "B.Cu") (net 2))
 (segment (start 166.413 64.699) (end 166.871187 64.699) (width 0.4064) (layer "B.Cu") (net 15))
 (segment (start 148.59 113.792) (end 132.283399 113.792) (width 0.4064) (layer "B.Cu") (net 15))
 (segment (start 168.656 76.2) (end 148.59 96.266) (width 0.4064) (layer "B.Cu") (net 15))
 (segment (start 132.283399 113.792) (end 129.99556 111.504161) (width 0.4064) (layer "B.Cu") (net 15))
 (segment (start 168.656 66.483813) (end 168.656 76.2) (width 0.4064) (layer "B.Cu") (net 15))
 (segment (start 166.871187 64.699) (end 168.656 66.483813) (width 0.4064) (layer "B.Cu") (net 15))
 (segment (start 148.59 96.266) (end 148.59 113.792) (width 0.4064) (layer "B.Cu") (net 15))
 (segment (start 135.07556 106.22444) (end 135.07556 111.504161) (width 0.4064) (layer "B.Cu") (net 16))
 (segment (start 157.663 73.449) (end 157.663 83.637) (width 0.4064) (layer "B.Cu") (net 16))
 (segment (start 157.663 83.637) (end 135.07556 106.22444) (width 0.4064) (layer "B.Cu") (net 16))
 (segment (start 104.394 80.01) (end 104.394 86.303001) (width 0.4064) (layer "B.Cu") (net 1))
 (segment (start 104.394 86.303001) (end 102.05284 88.644161) (width 0.4064) (layer "B.Cu") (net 1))
 (segment (start 97.026161 111.504161) (end 99.51556 111.504161) (width 0.4064) (layer "B.Cu") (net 3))
 (segment (start 104.356 59.658) (end 118.656 59.658) (width 0.4064) (layer "B.Cu") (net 3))
 (segment (start 78.74 93.218) (end 97.026161 111.504161) (width 0.4064) (layer "B.Cu") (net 3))
 (segment (start 118.656 59.658) (end 127.724 59.658) (width 0.4064) (layer "B.Cu") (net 3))
 (segment (start 146.304 59.658) (end 146.304 74.845) (width 0.4064) (layer "B.Cu") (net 3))
 (segment (start 127.724 59.658) (end 142.024 59.658) (width 0.4064) (layer "B.Cu") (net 3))
 (segment (start 142.024 59.658) (end 145.796 59.658) (width 0.4064) (layer "B.Cu") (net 3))
 (segment (start 82.912 62.63) (end 78.74 66.802) (width 0.4064) (layer "B.Cu") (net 3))
 (segment (start 158.274 59.658) (end 161.798 56.134) (width 0.4064) (layer "B.Cu") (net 3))
 (segment (start 165.1 56.134) (end 166.413 57.447) (width 0.4064) (layer "B.Cu") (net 3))
 (segment (start 78.74 66.802) (end 78.74 93.218) (width 0.4064) (layer "B.Cu") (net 3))
 (segment (start 166.413 57.447) (end 166.413 62.699) (width 0.4064) (layer "B.Cu") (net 3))
 (segment (start 145.796 59.658) (end 146.304 59.658) (width 0.4064) (layer "B.Cu") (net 3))
 (segment (start 101.384 62.63) (end 104.356 59.658) (width 0.4064) (layer "B.Cu") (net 3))
 (segment (start 98.78 62.63) (end 82.912 62.63) (width 0.4064) (layer "B.Cu") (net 3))
 (segment (start 146.304 59.658) (end 158.274 59.658) (width 0.4064) (layer "B.Cu") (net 3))
 (segment (start 98.78 62.63) (end 101.384 62.63) (width 0.4064) (layer "B.Cu") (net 3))
 (segment (start 161.798 56.134) (end 165.1 56.134) (width 0.4064) (layer "B.Cu") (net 3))
 (segment (start 146.304 74.845) (end 143.793 77.356) (width 0.4064) (layer "B.Cu") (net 3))
 (segment (start 109.474 83.763001) (end 104.59284 88.644161) (width 0.4064) (layer "B.Cu") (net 21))
 (segment (start 109.474 80.01) (end 109.474 83.763001) (width 0.4064) (layer "B.Cu") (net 21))
 (segment (start 114.554 80.01) (end 114.554 86.303001) (width 0.4064) (layer "B.Cu") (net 24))
 (segment (start 114.554 86.303001) (end 112.21284 88.644161) (width 0.4064) (layer "B.Cu") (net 24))
 (segment (start 119.634 86.303001) (end 117.29284 88.644161) (width 0.4064) (layer "B.Cu") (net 25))
 (segment (start 119.634 80.01) (end 119.634 86.303001) (width 0.4064) (layer "B.Cu") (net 25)))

